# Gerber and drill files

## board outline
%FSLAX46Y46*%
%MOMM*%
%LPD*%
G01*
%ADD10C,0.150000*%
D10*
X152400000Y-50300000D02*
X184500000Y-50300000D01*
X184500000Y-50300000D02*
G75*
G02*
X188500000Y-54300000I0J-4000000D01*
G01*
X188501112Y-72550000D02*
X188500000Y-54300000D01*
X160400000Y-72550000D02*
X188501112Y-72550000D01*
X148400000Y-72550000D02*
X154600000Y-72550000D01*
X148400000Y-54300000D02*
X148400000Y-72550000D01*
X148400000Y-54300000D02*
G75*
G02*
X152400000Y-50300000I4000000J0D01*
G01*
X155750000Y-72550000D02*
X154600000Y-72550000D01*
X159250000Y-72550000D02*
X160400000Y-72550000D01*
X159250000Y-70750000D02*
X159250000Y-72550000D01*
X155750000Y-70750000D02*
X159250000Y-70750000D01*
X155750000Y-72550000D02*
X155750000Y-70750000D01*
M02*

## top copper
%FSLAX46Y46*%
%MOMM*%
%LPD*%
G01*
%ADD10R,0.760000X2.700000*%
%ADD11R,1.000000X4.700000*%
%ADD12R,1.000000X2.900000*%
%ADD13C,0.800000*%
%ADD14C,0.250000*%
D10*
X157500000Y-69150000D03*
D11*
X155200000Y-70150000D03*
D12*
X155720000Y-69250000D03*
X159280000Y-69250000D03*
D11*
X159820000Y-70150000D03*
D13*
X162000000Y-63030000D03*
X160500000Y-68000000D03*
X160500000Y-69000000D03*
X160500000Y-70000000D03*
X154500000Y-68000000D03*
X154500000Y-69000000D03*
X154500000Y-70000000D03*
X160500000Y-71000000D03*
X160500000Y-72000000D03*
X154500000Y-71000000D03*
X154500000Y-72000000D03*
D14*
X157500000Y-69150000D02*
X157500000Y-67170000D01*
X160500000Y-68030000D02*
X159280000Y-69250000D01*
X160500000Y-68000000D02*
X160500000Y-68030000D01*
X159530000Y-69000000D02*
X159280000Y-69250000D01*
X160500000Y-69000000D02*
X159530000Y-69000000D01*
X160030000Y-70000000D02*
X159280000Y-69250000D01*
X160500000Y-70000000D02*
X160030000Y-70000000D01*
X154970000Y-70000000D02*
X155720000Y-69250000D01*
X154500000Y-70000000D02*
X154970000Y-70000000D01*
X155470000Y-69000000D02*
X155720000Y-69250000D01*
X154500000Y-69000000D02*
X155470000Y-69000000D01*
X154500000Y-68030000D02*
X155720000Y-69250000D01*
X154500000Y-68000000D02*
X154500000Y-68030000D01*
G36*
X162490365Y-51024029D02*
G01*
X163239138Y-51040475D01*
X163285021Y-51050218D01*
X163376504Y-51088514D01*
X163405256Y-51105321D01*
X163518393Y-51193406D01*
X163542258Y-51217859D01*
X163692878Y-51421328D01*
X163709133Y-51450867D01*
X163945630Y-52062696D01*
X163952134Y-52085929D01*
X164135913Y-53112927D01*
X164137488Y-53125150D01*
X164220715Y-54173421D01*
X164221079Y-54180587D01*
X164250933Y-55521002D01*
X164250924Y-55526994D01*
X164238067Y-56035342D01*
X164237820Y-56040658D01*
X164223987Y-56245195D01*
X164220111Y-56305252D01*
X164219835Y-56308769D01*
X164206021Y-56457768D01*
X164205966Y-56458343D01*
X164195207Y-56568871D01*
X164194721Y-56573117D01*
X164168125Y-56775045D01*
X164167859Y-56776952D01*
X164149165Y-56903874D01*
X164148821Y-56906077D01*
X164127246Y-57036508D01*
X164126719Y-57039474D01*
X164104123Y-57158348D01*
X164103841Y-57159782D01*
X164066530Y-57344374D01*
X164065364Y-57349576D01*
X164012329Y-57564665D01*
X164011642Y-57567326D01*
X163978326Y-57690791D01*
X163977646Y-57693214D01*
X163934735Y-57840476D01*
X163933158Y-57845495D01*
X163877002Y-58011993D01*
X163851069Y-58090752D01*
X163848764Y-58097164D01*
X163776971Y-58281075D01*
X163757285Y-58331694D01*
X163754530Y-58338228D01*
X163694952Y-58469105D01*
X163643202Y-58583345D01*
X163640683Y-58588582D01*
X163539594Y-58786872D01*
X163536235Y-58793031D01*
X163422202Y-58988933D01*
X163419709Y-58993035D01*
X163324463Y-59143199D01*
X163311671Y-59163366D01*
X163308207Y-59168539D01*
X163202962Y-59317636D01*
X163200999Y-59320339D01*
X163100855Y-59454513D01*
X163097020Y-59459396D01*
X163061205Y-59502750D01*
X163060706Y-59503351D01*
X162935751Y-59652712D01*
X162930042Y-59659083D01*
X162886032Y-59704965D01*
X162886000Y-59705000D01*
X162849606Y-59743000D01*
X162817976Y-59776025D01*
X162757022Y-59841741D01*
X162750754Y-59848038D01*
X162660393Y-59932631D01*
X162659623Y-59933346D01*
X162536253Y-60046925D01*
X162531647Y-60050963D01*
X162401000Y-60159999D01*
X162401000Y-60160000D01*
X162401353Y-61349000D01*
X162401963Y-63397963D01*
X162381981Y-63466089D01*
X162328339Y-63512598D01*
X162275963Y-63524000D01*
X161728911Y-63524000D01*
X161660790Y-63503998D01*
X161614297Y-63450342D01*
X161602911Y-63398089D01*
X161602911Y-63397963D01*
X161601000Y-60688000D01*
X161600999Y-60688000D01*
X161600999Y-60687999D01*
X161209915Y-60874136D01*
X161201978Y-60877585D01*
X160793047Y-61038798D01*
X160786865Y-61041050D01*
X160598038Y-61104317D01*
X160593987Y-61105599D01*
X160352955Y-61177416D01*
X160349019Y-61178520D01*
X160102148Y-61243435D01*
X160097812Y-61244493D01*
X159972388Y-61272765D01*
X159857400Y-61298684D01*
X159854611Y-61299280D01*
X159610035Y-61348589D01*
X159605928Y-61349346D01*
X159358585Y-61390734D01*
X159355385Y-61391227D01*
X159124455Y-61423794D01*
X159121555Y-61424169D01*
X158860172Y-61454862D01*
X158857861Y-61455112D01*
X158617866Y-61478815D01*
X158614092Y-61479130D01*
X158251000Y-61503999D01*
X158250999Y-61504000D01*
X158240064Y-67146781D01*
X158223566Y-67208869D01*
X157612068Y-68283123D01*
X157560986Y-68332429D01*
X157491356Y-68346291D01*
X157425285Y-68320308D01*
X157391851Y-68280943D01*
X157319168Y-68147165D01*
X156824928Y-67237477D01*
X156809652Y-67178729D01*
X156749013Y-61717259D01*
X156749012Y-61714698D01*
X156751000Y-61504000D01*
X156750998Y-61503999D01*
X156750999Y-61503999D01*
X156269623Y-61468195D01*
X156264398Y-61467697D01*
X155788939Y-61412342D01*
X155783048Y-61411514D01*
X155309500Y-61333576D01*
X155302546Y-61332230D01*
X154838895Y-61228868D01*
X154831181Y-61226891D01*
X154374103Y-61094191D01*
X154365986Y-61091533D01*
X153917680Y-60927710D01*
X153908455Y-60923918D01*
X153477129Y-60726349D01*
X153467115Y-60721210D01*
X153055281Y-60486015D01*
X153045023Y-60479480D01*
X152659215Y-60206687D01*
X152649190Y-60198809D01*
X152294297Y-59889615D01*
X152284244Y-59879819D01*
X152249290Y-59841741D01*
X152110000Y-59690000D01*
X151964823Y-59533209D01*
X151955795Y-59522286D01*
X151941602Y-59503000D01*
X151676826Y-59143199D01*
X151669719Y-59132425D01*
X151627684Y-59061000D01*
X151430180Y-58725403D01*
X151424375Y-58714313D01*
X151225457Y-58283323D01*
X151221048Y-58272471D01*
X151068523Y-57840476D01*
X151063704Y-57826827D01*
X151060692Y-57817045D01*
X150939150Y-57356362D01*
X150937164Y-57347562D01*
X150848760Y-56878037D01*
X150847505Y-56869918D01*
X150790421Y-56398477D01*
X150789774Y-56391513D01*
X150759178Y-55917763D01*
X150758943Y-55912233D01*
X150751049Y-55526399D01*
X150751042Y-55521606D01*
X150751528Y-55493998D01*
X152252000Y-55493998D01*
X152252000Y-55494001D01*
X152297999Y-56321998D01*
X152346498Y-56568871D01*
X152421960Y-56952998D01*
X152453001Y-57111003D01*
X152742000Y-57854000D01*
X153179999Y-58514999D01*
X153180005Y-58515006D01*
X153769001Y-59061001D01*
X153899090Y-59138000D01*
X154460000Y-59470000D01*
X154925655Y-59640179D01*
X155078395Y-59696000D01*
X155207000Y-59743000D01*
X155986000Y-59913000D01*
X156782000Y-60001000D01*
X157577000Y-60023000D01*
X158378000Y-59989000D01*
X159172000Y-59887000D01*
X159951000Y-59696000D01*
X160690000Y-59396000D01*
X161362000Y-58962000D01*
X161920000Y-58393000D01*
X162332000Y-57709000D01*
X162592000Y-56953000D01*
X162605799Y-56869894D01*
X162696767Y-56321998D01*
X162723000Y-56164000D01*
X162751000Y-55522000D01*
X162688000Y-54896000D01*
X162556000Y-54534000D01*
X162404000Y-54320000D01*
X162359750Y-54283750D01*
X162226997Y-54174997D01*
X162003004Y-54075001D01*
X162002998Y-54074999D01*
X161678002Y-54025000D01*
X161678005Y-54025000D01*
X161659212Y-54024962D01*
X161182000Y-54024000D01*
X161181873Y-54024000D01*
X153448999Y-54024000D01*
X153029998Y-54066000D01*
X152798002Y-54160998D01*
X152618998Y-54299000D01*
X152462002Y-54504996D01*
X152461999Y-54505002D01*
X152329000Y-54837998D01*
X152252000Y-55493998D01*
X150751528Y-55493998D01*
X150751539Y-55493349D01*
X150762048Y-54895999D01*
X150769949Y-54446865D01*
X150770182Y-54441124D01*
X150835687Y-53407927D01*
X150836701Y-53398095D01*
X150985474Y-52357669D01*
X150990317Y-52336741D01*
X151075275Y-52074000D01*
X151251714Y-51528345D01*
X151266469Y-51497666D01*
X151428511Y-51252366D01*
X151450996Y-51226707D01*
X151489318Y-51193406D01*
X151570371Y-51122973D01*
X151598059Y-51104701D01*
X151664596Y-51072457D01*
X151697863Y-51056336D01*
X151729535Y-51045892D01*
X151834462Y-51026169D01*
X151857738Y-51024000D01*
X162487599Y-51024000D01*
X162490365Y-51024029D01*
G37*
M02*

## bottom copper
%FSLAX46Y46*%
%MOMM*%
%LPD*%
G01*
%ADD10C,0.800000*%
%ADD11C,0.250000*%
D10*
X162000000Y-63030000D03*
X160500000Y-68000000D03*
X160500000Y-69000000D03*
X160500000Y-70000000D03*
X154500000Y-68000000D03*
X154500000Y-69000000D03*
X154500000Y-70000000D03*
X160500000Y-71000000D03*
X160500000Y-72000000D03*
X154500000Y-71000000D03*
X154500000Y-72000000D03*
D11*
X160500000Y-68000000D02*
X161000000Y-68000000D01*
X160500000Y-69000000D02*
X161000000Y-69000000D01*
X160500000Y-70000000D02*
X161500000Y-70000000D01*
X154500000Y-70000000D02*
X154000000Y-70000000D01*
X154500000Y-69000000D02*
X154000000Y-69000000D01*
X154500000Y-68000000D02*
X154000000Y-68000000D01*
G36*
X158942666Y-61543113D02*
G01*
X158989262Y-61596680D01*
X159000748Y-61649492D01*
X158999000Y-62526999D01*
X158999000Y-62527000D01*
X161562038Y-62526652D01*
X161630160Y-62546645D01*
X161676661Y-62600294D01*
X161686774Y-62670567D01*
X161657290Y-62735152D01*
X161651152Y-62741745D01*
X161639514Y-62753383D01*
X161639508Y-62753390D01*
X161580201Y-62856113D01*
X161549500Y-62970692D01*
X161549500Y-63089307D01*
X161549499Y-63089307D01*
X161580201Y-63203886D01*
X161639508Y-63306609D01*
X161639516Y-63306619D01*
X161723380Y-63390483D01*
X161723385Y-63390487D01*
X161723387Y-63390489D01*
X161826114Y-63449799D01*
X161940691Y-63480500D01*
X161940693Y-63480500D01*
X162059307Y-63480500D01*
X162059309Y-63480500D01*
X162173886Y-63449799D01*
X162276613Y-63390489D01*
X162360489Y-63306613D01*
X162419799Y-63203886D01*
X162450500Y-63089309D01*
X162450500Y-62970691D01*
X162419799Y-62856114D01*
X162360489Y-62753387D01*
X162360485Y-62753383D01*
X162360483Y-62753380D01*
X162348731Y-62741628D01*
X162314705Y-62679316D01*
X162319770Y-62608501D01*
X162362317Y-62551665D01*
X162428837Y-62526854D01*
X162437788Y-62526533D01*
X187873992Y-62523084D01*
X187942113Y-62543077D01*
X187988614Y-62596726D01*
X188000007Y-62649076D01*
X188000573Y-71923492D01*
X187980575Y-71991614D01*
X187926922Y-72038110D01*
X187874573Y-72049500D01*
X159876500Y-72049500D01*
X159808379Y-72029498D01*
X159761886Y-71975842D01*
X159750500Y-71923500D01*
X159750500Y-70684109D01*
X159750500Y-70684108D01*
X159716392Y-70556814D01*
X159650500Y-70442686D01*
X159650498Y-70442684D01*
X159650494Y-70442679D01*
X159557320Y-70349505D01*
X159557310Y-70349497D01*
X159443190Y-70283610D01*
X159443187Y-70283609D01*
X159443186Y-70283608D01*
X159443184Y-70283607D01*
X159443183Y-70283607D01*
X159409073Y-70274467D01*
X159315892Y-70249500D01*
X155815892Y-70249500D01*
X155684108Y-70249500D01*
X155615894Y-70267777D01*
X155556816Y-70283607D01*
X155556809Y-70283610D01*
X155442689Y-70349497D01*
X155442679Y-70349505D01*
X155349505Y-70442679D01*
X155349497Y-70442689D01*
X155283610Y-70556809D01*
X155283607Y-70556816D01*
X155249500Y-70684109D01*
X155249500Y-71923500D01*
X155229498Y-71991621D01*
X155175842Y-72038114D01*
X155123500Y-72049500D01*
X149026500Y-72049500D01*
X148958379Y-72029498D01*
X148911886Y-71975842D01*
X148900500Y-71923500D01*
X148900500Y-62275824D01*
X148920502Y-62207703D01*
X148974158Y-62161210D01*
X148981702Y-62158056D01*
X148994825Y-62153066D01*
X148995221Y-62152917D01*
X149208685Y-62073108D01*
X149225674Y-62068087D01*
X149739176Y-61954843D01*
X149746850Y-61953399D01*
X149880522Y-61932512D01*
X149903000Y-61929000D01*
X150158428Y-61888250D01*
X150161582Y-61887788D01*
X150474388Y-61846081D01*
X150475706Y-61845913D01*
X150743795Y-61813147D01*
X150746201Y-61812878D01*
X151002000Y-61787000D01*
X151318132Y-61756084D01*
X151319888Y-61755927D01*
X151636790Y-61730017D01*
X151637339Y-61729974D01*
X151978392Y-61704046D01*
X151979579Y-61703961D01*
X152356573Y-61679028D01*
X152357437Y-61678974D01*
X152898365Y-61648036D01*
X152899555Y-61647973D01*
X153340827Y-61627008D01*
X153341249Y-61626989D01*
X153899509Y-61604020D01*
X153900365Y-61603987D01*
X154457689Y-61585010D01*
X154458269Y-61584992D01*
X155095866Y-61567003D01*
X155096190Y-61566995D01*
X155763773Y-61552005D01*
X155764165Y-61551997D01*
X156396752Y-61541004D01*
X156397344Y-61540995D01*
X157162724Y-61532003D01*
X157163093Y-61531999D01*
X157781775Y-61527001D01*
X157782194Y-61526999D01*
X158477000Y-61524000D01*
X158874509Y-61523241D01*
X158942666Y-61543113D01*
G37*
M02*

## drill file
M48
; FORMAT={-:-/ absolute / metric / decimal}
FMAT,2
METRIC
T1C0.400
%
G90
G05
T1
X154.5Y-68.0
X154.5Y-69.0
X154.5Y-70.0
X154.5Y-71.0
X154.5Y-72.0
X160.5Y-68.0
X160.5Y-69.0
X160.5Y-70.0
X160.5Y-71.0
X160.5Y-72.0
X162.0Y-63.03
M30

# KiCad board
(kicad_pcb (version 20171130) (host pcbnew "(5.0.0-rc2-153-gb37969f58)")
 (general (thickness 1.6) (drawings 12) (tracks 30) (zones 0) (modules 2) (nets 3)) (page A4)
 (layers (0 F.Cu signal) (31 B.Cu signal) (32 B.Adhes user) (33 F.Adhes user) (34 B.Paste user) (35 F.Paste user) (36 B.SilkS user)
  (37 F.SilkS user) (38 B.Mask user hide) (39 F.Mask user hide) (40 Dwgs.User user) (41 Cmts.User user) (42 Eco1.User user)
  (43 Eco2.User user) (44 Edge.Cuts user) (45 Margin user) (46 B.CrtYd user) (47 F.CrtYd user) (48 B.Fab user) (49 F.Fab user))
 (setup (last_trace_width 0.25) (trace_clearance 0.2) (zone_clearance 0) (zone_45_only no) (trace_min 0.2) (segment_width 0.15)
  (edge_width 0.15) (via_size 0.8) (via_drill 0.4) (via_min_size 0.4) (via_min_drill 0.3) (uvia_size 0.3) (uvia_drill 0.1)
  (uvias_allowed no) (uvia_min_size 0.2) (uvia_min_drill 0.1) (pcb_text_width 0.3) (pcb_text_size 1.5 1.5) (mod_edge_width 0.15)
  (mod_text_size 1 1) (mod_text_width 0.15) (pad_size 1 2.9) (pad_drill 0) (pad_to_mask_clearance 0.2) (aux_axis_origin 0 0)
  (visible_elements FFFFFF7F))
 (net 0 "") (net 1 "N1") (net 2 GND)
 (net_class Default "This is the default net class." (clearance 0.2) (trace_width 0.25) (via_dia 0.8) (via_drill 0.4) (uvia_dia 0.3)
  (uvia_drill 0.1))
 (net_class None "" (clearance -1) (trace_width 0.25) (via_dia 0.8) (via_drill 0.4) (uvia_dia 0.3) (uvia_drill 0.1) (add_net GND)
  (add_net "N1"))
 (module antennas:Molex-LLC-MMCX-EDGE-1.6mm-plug (layer F.Cu) (at 157.5 69.75 180)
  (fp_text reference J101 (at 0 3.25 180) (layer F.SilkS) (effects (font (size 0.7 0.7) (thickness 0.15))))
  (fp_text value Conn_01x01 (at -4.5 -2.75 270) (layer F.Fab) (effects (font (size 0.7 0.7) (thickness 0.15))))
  (fp_line (start 1.75 -2.8) (end 2.9 -2.8) (layer Edge.Cuts) (width 0.15))
  (fp_line (start -1.75 -2.8) (end -2.9 -2.8) (layer Edge.Cuts) (width 0.15))
  (fp_line (start -1.75 -1) (end -1.75 -2.8) (layer Edge.Cuts) (width 0.15))
  (fp_line (start 1.75 -1) (end -1.75 -1) (layer Edge.Cuts) (width 0.15))
  (fp_line (start 1.75 -2.8) (end 1.75 -1) (layer Edge.Cuts) (width 0.15))
  (pad 1 smd rect (at 0 0.6 180) (size 0.76 2.7) (layers F.Cu F.Paste F.Mask) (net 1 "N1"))
  (pad 2 smd rect (at 2.3 -0.4 180) (size 1 4.7) (layers F.Cu F.Paste F.Mask) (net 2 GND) (zone_connect 2))
  (pad 2 smd rect (at 1.78 0.5 180) (size 1 2.9) (layers F.Cu F.Paste F.Mask) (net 2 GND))
  (pad 3 connect rect (at 0.83 0.55 180) (size 0.89 1) (layers Dwgs.User))
  (pad 2 smd rect (at -1.78 0.5 180) (size 1 2.9) (layers F.Cu F.Paste F.Mask) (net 2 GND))
  (pad 2 smd rect (at -2.32 -0.4 180) (size 1 4.7) (layers F.Cu F.Paste F.Mask) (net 2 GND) (zone_connect 2))
  (pad 3 connect rect (at -0.83 0.57 180) (size 0.89 1) (layers Dwgs.User)))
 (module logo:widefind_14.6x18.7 (layer F.Cu) (at 177.2 61.65)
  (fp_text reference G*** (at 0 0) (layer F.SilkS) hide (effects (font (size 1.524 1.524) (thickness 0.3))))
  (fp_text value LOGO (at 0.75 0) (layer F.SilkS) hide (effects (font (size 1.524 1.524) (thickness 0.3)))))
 (gr_line (start 152.4 50.3) (end 184.5 50.3) (layer Edge.Cuts) (width 0.15))
 (gr_arc (start 184.5 54.3) (end 188.5 54.3) (angle -90) (layer Edge.Cuts) (width 0.15))
 (gr_line (start 188.501112 72.55) (end 188.5 54.3) (layer Edge.Cuts) (width 0.15))
 (gr_line (start 160.4 72.55) (end 188.501112 72.55) (layer Edge.Cuts) (width 0.15))
 (gr_line (start 148.4 72.55) (end 154.6 72.55) (layer Edge.Cuts) (width 0.15))
 (gr_line (start 148.4 54.3) (end 148.4 72.55) (layer Edge.Cuts) (width 0.15))
 (gr_arc (start 152.4 54.3) (end 152.4 50.3) (angle -90) (layer Edge.Cuts) (width 0.15))
 (via (at 162 63.03) (size 0.8) (drill 0.4) (layers F.Cu B.Cu) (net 1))
 (segment (start 157.5 69.15) (end 157.5 67.17) (width 0.25) (layer F.Cu) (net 1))
 (via (at 160.5 68) (size 0.8) (drill 0.4) (layers F.Cu B.Cu) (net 2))
 (via (at 160.5 69) (size 0.8) (drill 0.4) (layers F.Cu B.Cu) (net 2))
 (via (at 160.5 70) (size 0.8) (drill 0.4) (layers F.Cu B.Cu) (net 2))
 (via (at 154.5 68) (size 0.8) (drill 0.4) (layers F.Cu B.Cu) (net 2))
 (via (at 154.5 69) (size 0.8) (drill 0.4) (layers F.Cu B.Cu) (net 2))
 (via (at 154.5 70) (size 0.8) (drill 0.4) (layers F.Cu B.Cu) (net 2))
 (segment (start 160.5 68.03) (end 159.28 69.25) (width 0.25) (layer F.Cu) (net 2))
 (segment (start 160.5 68) (end 160.5 68.03) (width 0.25) (layer F.Cu) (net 2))
 (segment (start 159.53 69) (end 159.28 69.25) (width 0.25) (layer F.Cu) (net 2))
 (segment (start 160.5 69) (end 159.53 69) (width 0.25) (layer F.Cu) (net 2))
 (segment (start 160.03 70) (end 159.28 69.25) (width 0.25) (layer F.Cu) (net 2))
 (segment (start 160.5 70) (end 160.03 70) (width 0.25) (layer F.Cu) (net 2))
 (segment (start 154.97 70) (end 155.72 69.25) (width 0.25) (layer F.Cu) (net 2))
 (segment (start 154.5 70) (end 154.97 70) (width 0.25) (layer F.Cu) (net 2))
 (segment (start 155.47 69) (end 155.72 69.25) (width 0.25) (layer F.Cu) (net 2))
 (segment (start 154.5 69) (end 155.47 69) (width 0.25) (layer F.Cu) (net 2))
 (segment (start 154.5 68.03) (end 155.72 69.25) (width 0.25) (layer F.Cu) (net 2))
 (segment (start 154.5 68) (end 154.5 68.03) (width 0.25) (layer F.Cu) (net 2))
 (segment (start 160.5 68) (end 161 68) (width 0.25) (layer B.Cu) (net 2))
 (segment (start 160.5 69) (end 161 69) (width 0.25) (layer B.Cu) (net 2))
 (segment (start 160.5 70) (end 161.5 70) (width 0.25) (layer B.Cu) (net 2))
 (segment (start 154.5 70) (end 154 70) (width 0.25) (layer B.Cu) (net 2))
 (segment (start 154.5 69) (end 154 69) (width 0.25) (layer B.Cu) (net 2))
 (segment (start 154.5 68) (end 154 68) (width 0.25) (layer B.Cu) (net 2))
 (via (at 160.5 71) (size 0.8) (drill 0.4) (layers F.Cu B.Cu) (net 2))
 (via (at 160.5 72) (size 0.8) (drill 0.4) (layers F.Cu B.Cu) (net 2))
 (via (at 154.5 71) (size 0.8) (drill 0.4) (layers F.Cu B.Cu) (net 2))
 (via (at 154.5 72) (size 0.8) (drill 0.4) (layers F.Cu B.Cu) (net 2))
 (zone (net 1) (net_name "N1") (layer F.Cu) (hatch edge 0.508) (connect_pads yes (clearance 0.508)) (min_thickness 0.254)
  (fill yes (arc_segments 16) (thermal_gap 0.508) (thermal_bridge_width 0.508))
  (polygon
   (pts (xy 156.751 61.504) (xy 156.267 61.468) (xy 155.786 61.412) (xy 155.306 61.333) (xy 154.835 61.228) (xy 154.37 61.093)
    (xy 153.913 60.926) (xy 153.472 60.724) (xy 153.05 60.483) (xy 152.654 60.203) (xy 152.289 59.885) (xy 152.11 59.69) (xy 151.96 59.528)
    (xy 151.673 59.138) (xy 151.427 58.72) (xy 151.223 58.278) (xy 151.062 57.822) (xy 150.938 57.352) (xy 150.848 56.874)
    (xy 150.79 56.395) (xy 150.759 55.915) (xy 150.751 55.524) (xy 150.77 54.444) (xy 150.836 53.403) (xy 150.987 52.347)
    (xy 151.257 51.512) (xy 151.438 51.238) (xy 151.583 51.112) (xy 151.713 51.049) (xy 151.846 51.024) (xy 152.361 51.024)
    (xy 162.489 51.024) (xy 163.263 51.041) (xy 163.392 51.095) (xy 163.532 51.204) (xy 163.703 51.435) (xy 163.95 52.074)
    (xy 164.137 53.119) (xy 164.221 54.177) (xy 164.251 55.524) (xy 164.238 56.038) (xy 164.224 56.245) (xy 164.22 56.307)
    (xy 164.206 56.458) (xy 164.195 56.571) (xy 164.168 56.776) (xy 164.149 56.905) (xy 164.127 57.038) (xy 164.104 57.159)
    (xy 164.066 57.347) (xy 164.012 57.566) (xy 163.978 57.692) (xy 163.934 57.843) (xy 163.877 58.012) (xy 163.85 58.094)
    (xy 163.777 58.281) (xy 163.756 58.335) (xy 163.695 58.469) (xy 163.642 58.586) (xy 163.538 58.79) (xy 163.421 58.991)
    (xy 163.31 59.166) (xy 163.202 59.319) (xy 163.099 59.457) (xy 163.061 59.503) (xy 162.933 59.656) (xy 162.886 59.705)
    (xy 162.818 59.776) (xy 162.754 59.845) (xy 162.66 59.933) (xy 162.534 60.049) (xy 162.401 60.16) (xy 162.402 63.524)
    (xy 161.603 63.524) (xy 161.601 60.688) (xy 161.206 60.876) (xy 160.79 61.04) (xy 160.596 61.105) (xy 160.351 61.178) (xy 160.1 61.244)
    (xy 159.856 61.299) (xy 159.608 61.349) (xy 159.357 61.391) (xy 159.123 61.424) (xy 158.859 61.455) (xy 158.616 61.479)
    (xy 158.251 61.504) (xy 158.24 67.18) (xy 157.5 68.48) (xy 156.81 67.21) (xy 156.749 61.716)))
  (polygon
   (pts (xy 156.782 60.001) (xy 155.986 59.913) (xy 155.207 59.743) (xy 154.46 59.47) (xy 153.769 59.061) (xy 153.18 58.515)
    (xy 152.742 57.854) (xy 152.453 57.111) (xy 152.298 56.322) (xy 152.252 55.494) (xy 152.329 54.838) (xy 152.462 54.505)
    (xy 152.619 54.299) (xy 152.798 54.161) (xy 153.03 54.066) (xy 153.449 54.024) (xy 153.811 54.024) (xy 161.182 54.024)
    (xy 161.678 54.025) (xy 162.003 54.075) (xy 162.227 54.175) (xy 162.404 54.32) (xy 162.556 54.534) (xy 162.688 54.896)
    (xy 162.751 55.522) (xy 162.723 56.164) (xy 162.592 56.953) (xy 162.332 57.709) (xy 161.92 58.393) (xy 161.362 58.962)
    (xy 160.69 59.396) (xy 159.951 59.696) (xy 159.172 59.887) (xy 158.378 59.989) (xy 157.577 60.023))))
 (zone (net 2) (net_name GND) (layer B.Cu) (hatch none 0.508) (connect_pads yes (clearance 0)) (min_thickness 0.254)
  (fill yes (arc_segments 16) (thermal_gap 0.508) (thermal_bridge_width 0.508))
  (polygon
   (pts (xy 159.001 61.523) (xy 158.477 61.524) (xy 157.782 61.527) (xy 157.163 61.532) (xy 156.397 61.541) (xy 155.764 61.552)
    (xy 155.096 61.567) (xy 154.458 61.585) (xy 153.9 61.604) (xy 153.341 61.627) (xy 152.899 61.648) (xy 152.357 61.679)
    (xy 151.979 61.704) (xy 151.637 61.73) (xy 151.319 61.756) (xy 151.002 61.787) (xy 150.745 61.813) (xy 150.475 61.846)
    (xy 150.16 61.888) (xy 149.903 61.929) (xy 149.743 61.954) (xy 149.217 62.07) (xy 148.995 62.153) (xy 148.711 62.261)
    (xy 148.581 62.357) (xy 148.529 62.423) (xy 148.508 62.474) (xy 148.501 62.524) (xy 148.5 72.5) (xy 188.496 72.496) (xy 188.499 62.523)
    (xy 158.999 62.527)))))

